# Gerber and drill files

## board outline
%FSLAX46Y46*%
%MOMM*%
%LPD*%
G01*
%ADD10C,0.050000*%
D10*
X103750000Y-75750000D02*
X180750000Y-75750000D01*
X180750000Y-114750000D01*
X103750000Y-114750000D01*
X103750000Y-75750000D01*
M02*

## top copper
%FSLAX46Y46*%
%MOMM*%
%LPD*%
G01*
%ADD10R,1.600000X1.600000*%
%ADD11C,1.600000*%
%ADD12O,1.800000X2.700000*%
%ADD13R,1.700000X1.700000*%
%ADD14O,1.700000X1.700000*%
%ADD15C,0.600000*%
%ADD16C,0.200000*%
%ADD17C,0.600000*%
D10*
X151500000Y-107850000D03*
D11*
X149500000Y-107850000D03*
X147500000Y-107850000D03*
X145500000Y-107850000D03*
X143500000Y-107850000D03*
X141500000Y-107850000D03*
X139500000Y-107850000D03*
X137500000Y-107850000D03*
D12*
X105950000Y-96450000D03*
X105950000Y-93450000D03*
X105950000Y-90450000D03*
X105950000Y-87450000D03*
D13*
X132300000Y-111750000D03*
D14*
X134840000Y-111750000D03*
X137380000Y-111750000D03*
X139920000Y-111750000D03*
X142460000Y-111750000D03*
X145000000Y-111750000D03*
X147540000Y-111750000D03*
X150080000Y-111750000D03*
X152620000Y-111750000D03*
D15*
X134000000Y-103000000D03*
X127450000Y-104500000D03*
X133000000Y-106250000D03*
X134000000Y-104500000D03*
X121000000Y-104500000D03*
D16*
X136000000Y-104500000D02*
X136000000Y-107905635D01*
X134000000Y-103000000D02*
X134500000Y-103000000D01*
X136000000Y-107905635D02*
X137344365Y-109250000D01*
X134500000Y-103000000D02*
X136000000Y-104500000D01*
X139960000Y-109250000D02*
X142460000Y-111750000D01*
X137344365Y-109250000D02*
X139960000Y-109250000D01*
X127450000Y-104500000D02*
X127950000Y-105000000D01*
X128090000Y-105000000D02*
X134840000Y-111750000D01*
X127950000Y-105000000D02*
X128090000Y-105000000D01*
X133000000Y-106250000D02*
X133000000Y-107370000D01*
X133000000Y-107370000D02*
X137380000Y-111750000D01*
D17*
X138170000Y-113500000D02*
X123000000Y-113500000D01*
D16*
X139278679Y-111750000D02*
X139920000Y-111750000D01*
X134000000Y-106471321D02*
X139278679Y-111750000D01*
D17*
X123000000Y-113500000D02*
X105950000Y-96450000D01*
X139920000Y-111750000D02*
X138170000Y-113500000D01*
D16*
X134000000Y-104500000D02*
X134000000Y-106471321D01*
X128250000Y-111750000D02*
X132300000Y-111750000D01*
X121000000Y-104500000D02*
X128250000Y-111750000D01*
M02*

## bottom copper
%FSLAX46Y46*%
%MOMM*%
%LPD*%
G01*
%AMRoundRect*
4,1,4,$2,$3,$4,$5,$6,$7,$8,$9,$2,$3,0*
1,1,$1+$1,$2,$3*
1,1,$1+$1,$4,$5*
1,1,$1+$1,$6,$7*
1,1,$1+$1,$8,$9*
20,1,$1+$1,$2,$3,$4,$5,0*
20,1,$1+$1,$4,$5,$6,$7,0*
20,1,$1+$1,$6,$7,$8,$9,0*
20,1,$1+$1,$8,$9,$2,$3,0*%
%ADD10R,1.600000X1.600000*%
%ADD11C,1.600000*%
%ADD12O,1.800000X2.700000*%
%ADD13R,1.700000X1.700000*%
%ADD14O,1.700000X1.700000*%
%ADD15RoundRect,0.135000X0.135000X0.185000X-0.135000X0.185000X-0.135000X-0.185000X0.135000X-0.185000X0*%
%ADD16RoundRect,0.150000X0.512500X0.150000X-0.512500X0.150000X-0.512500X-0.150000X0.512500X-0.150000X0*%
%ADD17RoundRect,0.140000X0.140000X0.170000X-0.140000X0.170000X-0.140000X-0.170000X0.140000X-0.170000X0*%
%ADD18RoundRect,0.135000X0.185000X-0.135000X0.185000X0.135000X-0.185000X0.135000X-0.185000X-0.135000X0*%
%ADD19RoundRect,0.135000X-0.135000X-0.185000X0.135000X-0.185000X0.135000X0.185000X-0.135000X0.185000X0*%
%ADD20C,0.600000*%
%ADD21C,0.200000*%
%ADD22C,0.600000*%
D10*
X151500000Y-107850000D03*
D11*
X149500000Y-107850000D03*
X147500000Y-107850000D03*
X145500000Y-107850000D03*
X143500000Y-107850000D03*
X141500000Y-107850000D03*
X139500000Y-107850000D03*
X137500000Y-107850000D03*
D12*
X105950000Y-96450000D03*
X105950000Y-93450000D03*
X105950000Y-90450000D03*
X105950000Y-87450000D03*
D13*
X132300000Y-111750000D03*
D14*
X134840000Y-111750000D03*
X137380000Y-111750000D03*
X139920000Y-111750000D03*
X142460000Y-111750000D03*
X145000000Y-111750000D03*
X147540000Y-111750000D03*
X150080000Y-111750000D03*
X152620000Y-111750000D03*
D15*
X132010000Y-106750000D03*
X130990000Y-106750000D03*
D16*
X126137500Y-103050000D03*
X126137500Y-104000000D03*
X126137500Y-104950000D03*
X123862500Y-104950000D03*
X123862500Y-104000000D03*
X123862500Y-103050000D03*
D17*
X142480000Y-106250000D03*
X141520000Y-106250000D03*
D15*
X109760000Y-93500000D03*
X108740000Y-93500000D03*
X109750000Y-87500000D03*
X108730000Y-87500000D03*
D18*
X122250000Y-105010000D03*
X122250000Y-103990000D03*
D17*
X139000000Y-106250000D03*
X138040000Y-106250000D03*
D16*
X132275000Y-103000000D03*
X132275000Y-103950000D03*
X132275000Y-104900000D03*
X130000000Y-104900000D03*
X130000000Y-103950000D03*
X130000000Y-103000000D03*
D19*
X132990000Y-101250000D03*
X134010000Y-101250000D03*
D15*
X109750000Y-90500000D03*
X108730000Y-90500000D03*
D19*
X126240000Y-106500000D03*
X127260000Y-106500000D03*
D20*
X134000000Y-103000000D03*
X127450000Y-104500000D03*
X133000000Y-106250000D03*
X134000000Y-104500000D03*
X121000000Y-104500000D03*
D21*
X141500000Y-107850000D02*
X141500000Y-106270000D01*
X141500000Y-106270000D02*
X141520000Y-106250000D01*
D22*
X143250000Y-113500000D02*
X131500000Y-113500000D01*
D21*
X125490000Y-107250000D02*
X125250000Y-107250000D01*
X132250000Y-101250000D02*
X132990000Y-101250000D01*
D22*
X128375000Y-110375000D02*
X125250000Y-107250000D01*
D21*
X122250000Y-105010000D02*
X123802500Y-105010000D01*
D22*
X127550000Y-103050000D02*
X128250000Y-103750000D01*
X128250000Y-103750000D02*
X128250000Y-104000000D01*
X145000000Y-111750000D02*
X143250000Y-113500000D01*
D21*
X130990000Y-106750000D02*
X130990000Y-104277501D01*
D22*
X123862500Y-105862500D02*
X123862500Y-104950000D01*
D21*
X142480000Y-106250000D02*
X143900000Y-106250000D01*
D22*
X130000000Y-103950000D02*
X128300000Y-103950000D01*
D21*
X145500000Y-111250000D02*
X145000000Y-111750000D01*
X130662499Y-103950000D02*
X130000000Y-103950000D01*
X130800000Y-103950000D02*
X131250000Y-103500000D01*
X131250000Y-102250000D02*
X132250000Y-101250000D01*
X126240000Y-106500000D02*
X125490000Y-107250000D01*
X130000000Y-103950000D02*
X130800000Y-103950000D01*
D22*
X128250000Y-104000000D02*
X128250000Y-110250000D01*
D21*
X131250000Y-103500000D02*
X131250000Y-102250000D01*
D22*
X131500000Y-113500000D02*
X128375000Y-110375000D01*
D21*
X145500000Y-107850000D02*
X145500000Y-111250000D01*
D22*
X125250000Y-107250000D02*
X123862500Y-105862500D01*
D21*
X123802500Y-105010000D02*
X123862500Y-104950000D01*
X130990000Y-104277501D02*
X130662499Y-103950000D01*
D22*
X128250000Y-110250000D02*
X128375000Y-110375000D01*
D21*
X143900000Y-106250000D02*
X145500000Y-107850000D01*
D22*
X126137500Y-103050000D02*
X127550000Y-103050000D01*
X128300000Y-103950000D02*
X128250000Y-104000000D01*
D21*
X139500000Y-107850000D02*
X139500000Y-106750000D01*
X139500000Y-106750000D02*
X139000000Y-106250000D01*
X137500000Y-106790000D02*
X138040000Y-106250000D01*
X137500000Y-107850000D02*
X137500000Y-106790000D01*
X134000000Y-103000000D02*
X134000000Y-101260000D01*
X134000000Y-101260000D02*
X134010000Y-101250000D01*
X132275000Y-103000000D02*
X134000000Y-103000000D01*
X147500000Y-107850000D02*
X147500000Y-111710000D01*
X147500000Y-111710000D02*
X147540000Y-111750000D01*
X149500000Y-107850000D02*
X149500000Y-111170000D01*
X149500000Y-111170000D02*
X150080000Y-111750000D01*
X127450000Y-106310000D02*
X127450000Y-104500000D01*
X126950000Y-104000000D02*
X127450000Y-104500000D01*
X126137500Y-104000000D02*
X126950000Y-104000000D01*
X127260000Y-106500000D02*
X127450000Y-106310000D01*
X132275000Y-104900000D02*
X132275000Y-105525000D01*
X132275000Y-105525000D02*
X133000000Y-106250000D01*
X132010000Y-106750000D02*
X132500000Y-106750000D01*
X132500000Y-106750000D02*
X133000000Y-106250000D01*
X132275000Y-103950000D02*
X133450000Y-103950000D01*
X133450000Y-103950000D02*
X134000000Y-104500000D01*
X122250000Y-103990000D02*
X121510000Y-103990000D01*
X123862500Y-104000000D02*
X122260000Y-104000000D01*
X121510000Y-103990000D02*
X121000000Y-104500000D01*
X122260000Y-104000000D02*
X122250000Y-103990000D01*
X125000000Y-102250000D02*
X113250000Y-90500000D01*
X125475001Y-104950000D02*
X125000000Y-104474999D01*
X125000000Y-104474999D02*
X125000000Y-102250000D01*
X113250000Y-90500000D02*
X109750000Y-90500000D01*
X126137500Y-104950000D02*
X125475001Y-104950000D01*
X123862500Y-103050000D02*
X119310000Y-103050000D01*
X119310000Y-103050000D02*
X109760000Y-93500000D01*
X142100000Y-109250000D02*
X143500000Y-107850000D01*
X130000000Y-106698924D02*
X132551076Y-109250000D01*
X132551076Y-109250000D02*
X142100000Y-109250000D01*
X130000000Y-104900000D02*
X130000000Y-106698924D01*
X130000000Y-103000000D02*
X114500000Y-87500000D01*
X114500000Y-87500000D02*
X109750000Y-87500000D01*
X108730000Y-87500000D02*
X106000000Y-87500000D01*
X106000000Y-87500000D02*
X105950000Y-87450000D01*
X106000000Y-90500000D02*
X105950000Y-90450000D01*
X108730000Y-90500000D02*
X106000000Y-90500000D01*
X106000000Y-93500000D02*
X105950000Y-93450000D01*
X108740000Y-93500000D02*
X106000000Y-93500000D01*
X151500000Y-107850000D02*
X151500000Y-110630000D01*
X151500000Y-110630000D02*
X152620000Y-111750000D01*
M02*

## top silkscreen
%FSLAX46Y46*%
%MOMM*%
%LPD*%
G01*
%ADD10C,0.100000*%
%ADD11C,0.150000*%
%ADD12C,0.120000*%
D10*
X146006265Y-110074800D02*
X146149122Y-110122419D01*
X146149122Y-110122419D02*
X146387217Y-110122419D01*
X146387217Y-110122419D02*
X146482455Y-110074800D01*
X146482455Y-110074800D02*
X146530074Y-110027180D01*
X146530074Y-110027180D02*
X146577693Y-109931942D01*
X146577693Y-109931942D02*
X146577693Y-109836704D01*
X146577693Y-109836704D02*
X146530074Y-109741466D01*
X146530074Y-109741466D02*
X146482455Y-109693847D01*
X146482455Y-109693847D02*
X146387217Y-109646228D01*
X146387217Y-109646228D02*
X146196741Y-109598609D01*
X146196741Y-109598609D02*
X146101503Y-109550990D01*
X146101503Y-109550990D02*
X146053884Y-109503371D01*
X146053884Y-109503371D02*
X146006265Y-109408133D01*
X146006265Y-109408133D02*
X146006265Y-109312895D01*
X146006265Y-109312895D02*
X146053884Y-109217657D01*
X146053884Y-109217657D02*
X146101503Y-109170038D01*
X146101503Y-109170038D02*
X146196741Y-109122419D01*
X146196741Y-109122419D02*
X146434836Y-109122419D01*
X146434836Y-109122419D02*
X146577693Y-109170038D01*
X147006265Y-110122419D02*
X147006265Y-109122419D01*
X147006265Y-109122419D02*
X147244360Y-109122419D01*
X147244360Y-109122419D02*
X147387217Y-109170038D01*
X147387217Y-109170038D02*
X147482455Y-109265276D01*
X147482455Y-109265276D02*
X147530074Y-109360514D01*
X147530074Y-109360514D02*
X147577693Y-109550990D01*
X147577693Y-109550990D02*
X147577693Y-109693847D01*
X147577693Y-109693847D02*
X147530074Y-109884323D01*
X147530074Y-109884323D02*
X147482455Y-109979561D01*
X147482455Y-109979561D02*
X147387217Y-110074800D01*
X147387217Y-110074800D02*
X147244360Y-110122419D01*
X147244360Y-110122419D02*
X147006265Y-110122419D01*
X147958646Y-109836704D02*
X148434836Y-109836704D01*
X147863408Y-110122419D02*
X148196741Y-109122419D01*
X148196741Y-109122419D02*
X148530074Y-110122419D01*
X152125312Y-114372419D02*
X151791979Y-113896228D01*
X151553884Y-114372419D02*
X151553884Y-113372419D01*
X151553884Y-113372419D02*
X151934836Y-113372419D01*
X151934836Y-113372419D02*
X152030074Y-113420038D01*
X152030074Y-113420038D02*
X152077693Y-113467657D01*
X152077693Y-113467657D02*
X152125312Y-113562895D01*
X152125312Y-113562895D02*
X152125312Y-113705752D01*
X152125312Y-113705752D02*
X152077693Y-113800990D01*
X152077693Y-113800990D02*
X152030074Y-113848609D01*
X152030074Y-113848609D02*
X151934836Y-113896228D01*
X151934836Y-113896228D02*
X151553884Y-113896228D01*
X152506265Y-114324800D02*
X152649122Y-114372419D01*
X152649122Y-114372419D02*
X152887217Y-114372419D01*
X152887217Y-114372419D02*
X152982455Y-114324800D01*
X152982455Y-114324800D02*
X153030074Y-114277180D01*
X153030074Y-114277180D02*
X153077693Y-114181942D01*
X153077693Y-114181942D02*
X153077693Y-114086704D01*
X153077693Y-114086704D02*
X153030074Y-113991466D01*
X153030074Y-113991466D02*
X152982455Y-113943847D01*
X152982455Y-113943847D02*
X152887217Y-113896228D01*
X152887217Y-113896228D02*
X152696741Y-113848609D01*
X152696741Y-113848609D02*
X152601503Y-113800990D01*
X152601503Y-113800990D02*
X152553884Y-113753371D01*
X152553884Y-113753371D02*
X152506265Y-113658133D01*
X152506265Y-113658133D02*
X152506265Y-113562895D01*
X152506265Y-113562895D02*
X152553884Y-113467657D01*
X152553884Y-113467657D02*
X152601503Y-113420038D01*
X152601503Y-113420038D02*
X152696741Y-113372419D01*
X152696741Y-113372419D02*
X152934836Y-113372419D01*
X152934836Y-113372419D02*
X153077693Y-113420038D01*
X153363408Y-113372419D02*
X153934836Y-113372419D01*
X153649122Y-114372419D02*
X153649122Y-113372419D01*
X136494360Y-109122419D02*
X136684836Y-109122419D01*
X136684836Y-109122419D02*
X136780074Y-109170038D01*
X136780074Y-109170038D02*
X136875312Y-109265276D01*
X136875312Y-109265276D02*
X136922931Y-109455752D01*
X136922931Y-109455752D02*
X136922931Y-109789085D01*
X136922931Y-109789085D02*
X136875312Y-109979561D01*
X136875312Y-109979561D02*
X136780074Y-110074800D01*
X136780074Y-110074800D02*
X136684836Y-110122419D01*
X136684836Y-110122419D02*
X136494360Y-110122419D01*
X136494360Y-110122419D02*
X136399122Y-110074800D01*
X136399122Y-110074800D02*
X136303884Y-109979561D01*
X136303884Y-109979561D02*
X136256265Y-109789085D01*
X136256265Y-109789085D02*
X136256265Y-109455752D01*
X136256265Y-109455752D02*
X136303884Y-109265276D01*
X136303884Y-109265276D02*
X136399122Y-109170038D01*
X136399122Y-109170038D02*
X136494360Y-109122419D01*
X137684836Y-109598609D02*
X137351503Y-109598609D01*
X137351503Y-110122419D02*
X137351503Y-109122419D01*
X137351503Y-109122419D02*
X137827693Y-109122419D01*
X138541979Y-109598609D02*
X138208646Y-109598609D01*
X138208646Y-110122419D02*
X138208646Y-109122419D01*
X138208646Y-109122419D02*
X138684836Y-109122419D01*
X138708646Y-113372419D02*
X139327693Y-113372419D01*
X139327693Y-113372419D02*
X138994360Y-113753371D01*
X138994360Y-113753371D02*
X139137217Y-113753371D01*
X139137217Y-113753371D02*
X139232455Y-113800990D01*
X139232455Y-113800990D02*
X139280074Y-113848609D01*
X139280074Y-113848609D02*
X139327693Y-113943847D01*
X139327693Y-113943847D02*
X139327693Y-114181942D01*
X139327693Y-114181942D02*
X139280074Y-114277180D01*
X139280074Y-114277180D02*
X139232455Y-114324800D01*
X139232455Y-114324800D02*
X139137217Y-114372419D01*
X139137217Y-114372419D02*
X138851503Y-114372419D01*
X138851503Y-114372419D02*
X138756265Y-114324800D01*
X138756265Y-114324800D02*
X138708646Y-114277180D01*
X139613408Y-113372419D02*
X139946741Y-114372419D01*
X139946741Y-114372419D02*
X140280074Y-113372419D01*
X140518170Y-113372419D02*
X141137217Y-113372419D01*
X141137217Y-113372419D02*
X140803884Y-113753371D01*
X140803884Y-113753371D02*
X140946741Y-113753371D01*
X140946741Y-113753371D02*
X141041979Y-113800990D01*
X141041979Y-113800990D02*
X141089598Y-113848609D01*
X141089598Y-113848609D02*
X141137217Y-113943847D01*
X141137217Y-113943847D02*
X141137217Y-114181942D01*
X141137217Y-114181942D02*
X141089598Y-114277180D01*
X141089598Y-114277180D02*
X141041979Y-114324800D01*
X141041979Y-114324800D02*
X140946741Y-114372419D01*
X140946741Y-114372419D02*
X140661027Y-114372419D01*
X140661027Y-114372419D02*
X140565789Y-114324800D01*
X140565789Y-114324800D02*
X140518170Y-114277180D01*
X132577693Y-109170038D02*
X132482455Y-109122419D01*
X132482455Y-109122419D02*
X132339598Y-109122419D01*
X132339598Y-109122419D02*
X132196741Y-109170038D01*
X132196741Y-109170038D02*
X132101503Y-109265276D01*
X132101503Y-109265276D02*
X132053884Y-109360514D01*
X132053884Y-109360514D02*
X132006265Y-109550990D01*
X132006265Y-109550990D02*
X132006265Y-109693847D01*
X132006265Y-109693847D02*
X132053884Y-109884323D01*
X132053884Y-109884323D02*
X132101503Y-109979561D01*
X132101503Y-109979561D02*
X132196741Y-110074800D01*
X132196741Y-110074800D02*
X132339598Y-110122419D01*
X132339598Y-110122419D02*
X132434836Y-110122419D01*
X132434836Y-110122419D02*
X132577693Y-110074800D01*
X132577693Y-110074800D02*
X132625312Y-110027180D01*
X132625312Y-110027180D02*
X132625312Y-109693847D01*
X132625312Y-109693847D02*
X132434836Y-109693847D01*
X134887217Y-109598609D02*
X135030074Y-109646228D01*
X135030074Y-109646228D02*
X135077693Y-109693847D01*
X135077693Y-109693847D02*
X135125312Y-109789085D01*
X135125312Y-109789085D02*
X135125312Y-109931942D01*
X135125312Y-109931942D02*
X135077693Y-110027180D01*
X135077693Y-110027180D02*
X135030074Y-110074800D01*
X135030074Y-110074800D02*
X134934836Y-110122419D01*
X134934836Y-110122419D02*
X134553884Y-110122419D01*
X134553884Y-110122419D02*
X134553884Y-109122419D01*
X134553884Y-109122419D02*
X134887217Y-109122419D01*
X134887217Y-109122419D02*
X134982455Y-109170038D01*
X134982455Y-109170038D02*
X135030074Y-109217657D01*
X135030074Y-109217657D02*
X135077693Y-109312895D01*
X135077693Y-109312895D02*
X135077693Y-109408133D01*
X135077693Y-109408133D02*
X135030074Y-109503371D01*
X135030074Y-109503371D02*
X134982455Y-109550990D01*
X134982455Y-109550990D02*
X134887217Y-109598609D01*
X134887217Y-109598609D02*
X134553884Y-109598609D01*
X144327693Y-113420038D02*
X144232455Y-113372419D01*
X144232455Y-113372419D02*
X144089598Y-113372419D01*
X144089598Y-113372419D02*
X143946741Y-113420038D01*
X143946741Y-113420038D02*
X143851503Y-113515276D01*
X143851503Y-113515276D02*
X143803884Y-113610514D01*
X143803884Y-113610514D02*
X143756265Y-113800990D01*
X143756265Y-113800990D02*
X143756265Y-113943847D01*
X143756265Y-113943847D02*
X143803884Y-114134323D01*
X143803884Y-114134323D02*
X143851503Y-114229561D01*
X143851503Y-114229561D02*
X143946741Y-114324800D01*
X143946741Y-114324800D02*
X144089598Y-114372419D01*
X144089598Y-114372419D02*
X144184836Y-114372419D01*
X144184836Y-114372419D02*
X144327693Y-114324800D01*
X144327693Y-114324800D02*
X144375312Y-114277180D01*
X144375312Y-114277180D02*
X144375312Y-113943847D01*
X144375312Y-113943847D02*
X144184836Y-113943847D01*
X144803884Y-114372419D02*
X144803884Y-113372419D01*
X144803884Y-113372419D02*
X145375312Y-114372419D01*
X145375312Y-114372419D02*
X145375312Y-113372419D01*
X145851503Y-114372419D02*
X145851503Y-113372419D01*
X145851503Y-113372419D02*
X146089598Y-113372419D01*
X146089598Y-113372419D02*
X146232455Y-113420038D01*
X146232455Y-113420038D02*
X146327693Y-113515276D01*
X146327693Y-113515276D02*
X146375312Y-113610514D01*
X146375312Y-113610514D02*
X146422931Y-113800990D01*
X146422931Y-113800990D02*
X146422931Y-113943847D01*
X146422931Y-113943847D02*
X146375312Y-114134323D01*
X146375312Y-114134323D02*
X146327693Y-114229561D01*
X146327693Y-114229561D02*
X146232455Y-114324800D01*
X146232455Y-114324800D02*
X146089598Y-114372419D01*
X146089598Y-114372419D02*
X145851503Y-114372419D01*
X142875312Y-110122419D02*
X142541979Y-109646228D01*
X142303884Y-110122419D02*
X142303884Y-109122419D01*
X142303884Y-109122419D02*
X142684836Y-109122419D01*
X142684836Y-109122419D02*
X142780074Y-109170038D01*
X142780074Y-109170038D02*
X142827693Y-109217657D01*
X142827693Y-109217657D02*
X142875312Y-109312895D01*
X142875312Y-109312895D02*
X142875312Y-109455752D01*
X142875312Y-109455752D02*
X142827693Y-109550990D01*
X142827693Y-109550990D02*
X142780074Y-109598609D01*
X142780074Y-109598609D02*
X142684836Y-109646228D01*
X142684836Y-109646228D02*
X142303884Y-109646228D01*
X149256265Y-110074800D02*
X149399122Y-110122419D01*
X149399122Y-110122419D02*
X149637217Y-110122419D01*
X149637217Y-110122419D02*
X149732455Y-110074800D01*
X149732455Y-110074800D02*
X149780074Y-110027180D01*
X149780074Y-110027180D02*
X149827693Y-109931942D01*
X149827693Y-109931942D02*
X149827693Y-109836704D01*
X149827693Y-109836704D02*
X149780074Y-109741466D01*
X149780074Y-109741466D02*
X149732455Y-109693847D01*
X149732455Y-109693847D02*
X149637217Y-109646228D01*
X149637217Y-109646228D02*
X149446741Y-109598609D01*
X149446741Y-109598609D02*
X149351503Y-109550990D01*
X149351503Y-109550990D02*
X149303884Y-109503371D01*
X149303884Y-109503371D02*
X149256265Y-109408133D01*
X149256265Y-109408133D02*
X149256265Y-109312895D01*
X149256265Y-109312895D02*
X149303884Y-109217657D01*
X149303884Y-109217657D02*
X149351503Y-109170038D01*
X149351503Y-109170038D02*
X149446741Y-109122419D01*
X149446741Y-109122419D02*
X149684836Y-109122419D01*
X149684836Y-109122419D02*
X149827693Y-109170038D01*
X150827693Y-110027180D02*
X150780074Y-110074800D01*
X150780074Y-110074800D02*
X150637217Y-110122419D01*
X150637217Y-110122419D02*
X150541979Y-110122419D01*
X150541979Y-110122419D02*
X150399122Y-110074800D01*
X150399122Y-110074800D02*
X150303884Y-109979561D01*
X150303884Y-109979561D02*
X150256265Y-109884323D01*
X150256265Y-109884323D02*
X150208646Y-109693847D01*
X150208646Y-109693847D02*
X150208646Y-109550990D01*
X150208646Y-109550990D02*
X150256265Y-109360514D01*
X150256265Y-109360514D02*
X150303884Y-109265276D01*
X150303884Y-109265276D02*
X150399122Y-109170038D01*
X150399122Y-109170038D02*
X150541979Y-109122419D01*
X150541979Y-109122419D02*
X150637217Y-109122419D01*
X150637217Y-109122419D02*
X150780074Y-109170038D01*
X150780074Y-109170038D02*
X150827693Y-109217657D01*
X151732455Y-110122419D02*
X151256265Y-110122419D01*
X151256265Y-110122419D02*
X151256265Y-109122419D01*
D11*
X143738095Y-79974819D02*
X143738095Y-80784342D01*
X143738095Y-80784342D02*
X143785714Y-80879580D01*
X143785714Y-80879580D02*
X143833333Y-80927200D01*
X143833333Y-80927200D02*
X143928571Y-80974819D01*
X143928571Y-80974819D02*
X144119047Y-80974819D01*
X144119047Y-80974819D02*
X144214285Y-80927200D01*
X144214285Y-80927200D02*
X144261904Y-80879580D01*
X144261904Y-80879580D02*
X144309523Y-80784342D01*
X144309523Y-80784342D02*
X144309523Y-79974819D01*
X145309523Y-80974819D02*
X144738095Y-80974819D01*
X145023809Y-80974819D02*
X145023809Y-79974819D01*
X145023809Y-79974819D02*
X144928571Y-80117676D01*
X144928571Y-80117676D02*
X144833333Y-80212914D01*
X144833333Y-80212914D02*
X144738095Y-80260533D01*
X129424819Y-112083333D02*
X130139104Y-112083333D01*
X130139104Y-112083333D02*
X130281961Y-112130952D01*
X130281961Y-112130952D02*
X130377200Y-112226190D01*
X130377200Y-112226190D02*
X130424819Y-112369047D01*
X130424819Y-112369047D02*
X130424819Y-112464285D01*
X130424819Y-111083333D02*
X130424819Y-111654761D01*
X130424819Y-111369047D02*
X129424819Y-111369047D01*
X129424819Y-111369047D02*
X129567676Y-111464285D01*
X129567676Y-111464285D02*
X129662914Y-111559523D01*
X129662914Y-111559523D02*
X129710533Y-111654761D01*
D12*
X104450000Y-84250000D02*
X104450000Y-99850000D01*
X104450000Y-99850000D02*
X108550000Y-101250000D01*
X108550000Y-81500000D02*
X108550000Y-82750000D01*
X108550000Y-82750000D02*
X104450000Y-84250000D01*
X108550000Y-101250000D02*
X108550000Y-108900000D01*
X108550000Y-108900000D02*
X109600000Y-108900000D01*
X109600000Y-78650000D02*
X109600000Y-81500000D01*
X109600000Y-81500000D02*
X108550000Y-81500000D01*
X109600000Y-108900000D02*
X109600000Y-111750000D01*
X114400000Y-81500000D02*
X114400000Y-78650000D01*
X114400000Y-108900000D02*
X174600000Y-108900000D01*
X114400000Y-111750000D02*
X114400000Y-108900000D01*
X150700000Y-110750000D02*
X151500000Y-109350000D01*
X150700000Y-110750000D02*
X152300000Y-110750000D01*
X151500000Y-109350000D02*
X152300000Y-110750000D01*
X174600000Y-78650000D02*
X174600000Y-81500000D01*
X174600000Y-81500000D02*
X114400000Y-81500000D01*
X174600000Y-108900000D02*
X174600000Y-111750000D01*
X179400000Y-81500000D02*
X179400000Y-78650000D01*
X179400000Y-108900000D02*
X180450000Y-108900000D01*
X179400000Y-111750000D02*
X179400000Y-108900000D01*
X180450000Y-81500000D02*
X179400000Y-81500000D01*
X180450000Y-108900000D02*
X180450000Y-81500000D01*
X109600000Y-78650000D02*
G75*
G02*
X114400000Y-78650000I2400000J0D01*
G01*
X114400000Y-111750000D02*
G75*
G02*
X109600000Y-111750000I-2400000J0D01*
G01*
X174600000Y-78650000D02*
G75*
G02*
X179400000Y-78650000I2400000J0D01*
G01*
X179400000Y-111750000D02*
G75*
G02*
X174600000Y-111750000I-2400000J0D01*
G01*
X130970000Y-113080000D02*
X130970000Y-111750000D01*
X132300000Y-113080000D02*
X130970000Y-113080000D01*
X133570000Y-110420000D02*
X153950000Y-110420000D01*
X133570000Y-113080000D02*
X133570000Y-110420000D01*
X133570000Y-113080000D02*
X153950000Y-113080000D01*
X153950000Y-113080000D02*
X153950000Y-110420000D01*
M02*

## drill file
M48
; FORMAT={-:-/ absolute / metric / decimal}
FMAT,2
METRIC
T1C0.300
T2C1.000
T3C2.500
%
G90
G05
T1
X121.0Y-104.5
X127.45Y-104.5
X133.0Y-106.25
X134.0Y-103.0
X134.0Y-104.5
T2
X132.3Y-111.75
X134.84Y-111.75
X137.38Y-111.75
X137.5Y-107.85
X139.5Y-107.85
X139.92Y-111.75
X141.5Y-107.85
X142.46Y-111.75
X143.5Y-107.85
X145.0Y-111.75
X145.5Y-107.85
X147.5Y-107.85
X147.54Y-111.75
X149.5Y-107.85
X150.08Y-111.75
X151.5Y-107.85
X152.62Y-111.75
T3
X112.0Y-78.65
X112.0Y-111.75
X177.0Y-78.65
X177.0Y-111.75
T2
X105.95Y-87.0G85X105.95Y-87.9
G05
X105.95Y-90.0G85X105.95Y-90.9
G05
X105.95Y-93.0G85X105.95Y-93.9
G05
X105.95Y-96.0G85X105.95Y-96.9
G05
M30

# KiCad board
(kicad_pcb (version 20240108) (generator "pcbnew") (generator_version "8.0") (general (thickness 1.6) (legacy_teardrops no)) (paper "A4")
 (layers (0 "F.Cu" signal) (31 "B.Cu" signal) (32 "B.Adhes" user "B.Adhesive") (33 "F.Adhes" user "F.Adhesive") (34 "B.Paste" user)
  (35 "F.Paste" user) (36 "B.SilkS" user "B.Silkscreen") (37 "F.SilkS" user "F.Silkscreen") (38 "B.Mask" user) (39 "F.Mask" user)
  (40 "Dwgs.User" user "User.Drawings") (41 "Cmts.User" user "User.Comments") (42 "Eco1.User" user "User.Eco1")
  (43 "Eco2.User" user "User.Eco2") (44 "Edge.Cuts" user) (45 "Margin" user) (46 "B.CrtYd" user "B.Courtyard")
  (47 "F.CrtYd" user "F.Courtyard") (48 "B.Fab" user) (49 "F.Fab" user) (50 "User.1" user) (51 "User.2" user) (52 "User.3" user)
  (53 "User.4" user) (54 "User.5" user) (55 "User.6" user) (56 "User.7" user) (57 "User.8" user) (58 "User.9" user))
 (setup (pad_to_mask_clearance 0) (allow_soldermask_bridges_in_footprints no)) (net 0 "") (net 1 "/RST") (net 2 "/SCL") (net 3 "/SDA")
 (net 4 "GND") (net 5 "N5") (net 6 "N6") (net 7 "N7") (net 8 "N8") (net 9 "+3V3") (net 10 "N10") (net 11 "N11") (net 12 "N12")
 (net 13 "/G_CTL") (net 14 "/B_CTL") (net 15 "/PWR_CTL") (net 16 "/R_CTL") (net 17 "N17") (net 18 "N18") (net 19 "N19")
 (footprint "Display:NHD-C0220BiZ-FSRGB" (layer "F.Cu") (at 144.5 91.95)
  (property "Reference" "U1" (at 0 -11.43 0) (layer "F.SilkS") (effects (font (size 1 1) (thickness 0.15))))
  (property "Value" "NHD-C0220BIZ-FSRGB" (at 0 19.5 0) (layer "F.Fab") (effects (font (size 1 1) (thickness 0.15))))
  (fp_line (start -40.05 -7.7) (end -40.05 7.9) (stroke (width 0.12) (type solid)) (layer "F.SilkS"))
  (fp_line (start -40.05 7.9) (end -35.95 9.3) (stroke (width 0.12) (type solid)) (layer "F.SilkS"))
  (fp_line (start -35.95 -10.45) (end -35.95 -9.2) (stroke (width 0.12) (type solid)) (layer "F.SilkS"))
  (fp_line (start -35.95 -9.2) (end -40.05 -7.7) (stroke (width 0.12) (type solid)) (layer "F.SilkS"))
  (fp_line (start -35.95 9.3) (end -35.95 16.95) (stroke (width 0.12) (type solid)) (layer "F.SilkS"))
  (fp_line (start -35.95 16.95) (end -34.9 16.95) (stroke (width 0.12) (type solid)) (layer "F.SilkS"))
  (fp_line (start -34.9 -13.3) (end -34.9 -10.45) (stroke (width 0.12) (type solid)) (layer "F.SilkS"))
  (fp_line (start -34.9 -10.45) (end -35.95 -10.45) (stroke (width 0.12) (type solid)) (layer "F.SilkS"))
  (fp_line (start -34.9 16.95) (end -34.9 19.8) (stroke (width 0.12) (type solid)) (layer "F.SilkS"))
  (fp_line (start -30.1 -10.45) (end -30.1 -13.3) (stroke (width 0.12) (type solid)) (layer "F.SilkS"))
  (fp_line (start -30.1 16.95) (end 30.1 16.95) (stroke (width 0.12) (type solid)) (layer "F.SilkS"))
  (fp_line (start -30.1 19.8) (end -30.1 16.95) (stroke (width 0.12) (type solid)) (layer "F.SilkS"))
  (fp_line (start 6.2 18.8) (end 7 17.4) (stroke (width 0.12) (type solid)) (layer "F.SilkS"))
  (fp_line (start 6.2 18.8) (end 7.8 18.8) (stroke (width 0.12) (type solid)) (layer "F.SilkS"))
  (fp_line (start 7 17.4) (end 7.8 18.8) (stroke (width 0.12) (type solid)) (layer "F.SilkS"))
  (fp_line (start 30.1 -13.3) (end 30.1 -10.45) (stroke (width 0.12) (type solid)) (layer "F.SilkS"))
  (fp_line (start 30.1 -10.45) (end -30.1 -10.45) (stroke (width 0.12) (type solid)) (layer "F.SilkS"))
  (fp_line (start 30.1 16.95) (end 30.1 19.8) (stroke (width 0.12) (type solid)) (layer "F.SilkS"))
  (fp_line (start 34.9 -10.45) (end 34.9 -13.3) (stroke (width 0.12) (type solid)) (layer "F.SilkS"))
  (fp_line (start 34.9 16.95) (end 35.95 16.95) (stroke (width 0.12) (type solid)) (layer "F.SilkS"))
  (fp_line (start 34.9 19.8) (end 34.9 16.95) (stroke (width 0.12) (type solid)) (layer "F.SilkS"))
  (fp_line (start 35.95 -10.45) (end 34.9 -10.45) (stroke (width 0.12) (type solid)) (layer "F.SilkS"))
  (fp_line (start 35.95 16.95) (end 35.95 -10.45) (stroke (width 0.12) (type solid)) (layer "F.SilkS"))
  (fp_arc (start -34.9 -13.3) (mid -32.5 -15.7) (end -30.1 -13.3) (stroke (width 0.12) (type solid)) (layer "F.SilkS"))
  (fp_arc (start -30.1 19.8) (mid -32.5 22.2) (end -34.9 19.8) (stroke (width 0.12) (type solid)) (layer "F.SilkS"))
  (fp_arc (start 30.1 -13.3) (mid 32.5 -15.7) (end 34.9 -13.3) (stroke (width 0.12) (type solid)) (layer "F.SilkS"))
  (fp_arc (start 34.9 19.8) (mid 32.5 22.2) (end 30.1 19.8) (stroke (width 0.12) (type solid)) (layer "F.SilkS"))
  (pad "" np_thru_hole circle (at -32.5 -13.3) (size 2.5 2.5) (drill 2.5) (layers "*.Cu" "*.Mask"))
  (pad "" np_thru_hole circle (at -32.5 19.8) (size 2.5 2.5) (drill 2.5) (layers "*.Cu" "*.Mask"))
  (pad "" np_thru_hole circle (at 32.5 -13.3) (size 2.5 2.5) (drill 2.5) (layers "*.Cu" "*.Mask"))
  (pad "" np_thru_hole circle (at 32.5 19.8) (size 2.5 2.5) (drill 2.5) (layers "*.Cu" "*.Mask"))
  (pad "1" thru_hole rect (at 7 15.9) (size 1.6 1.6) (drill 1) (layers "*.Cu" "*.Mask") (remove_unused_layers no) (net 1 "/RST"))
  (pad "2" thru_hole circle (at 5 15.9) (size 1.6 1.6) (drill 1) (layers "*.Cu" "*.Mask") (remove_unused_layers no) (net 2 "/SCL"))
  (pad "3" thru_hole circle (at 3 15.9) (size 1.6 1.6) (drill 1) (layers "*.Cu" "*.Mask") (remove_unused_layers no) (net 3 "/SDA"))
  (pad "4" thru_hole circle (at 1 15.9) (size 1.6 1.6) (drill 1) (layers "*.Cu" "*.Mask") (remove_unused_layers no) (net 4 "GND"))
  (pad "5" thru_hole circle (at -1 15.9) (size 1.6 1.6) (drill 1) (layers "*.Cu" "*.Mask") (remove_unused_layers no) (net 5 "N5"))
  (pad "6" thru_hole circle (at -3 15.9) (size 1.6 1.6) (drill 1) (layers "*.Cu" "*.Mask") (remove_unused_layers no) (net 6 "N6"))
  (pad "7" thru_hole circle (at -5 15.9) (size 1.6 1.6) (drill 1) (layers "*.Cu" "*.Mask") (remove_unused_layers no) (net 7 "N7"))
  (pad "8" thru_hole circle (at -7 15.9) (size 1.6 1.6) (drill 1) (layers "*.Cu" "*.Mask") (remove_unused_layers no) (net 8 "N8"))
  (pad "9" thru_hole oval (at -38.55 4.5) (size 1.8 2.7) (drill oval 1 1.9) (layers "*.Cu" "*.Mask") (remove_unused_layers no)
   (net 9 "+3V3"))
  (pad "10" thru_hole oval (at -38.55 1.5) (size 1.8 2.7) (drill oval 1 1.9) (layers "*.Cu" "*.Mask") (remove_unused_layers no)
   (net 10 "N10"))
  (pad "11" thru_hole oval (at -38.55 -1.5) (size 1.8 2.7) (drill oval 1 1.9) (layers "*.Cu" "*.Mask") (remove_unused_layers no)
   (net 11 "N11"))
  (pad "12" thru_hole oval (at -38.55 -4.5) (size 1.8 2.7) (drill oval 1 1.9) (layers "*.Cu" "*.Mask") (remove_unused_layers no)
   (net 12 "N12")))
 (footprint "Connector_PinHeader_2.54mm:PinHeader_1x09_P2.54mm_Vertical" (layer "F.Cu") (at 132.3 111.75 90)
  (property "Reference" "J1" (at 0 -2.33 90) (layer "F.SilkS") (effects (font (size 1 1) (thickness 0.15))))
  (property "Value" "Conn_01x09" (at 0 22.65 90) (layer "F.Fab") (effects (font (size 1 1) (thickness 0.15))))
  (fp_line (start -1.33 -1.33) (end 0 -1.33) (stroke (width 0.12) (type solid)) (layer "F.SilkS"))
  (fp_line (start -1.33 0) (end -1.33 -1.33) (stroke (width 0.12) (type solid)) (layer "F.SilkS"))
  (fp_line (start 1.33 1.27) (end 1.33 21.65) (stroke (width 0.12) (type solid)) (layer "F.SilkS"))
  (fp_line (start -1.33 1.27) (end 1.33 1.27) (stroke (width 0.12) (type solid)) (layer "F.SilkS"))
  (fp_line (start -1.33 1.27) (end -1.33 21.65) (stroke (width 0.12) (type solid)) (layer "F.SilkS"))
  (fp_line (start -1.33 21.65) (end 1.33 21.65) (stroke (width 0.12) (type solid)) (layer "F.SilkS"))
  (pad "1" thru_hole rect (at 0 0 90) (size 1.7 1.7) (drill 1) (layers "*.Cu" "*.Mask") (remove_unused_layers no) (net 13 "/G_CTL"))
  (pad "2" thru_hole oval (at 0 2.54 90) (size 1.7 1.7) (drill 1) (layers "*.Cu" "*.Mask") (remove_unused_layers no) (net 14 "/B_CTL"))
  (pad "3" thru_hole oval (at 0 5.08 90) (size 1.7 1.7) (drill 1) (layers "*.Cu" "*.Mask") (remove_unused_layers no) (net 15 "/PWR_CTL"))
  (pad "4" thru_hole oval (at 0 7.62 90) (size 1.7 1.7) (drill 1) (layers "*.Cu" "*.Mask") (remove_unused_layers no) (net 9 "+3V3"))
  (pad "5" thru_hole oval (at 0 10.16 90) (size 1.7 1.7) (drill 1) (layers "*.Cu" "*.Mask") (remove_unused_layers no) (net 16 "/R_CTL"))
  (pad "6" thru_hole oval (at 0 12.7 90) (size 1.7 1.7) (drill 1) (layers "*.Cu" "*.Mask") (remove_unused_layers no) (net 4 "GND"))
  (pad "7" thru_hole oval (at 0 15.24 90) (size 1.7 1.7) (drill 1) (layers "*.Cu" "*.Mask") (remove_unused_layers no) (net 3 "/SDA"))
  (pad "8" thru_hole oval (at 0 17.78 90) (size 1.7 1.7) (drill 1) (layers "*.Cu" "*.Mask") (remove_unused_layers no) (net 2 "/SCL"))
  (pad "9" thru_hole oval (at 0 20.32 90) (size 1.7 1.7) (drill 1) (layers "*.Cu" "*.Mask") (remove_unused_layers no) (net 1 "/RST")))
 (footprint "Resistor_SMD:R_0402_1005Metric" (layer "B.Cu") (at 131.5 106.75 180)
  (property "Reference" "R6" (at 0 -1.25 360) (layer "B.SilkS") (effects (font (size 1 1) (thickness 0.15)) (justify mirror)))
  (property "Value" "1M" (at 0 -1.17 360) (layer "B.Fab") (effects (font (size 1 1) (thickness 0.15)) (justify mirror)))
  (pad "1" smd roundrect (at -0.51 0 180) (size 0.54 0.64) (layers "B.Cu" "B.Paste" "B.Mask") (roundrect_rratio 0.25) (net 15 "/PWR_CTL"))
  (pad "2" smd roundrect (at 0.51 0 180) (size 0.54 0.64) (layers "B.Cu" "B.Paste" "B.Mask") (roundrect_rratio 0.25) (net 4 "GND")))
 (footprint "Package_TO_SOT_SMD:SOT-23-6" (layer "B.Cu") (at 125 104 180)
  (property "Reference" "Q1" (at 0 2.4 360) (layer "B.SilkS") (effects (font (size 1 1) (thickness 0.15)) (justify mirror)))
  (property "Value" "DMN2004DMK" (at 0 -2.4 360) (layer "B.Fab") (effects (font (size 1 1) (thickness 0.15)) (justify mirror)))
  (pad "1" smd roundrect (at -1.1375 0.95 180) (size 1.325 0.6) (layers "B.Cu" "B.Paste" "B.Mask") (roundrect_rratio 0.25) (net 4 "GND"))
  (pad "2" smd roundrect (at -1.1375 0 180) (size 1.325 0.6) (layers "B.Cu" "B.Paste" "B.Mask") (roundrect_rratio 0.25) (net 14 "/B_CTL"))
  (pad "3" smd roundrect (at -1.1375 -0.95 180) (size 1.325 0.6) (layers "B.Cu" "B.Paste" "B.Mask") (roundrect_rratio 0.25) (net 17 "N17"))
  (pad "4" smd roundrect (at 1.1375 -0.95 180) (size 1.325 0.6) (layers "B.Cu" "B.Paste" "B.Mask") (roundrect_rratio 0.25) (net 4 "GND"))
  (pad "5" smd roundrect (at 1.1375 0 180) (size 1.325 0.6) (layers "B.Cu" "B.Paste" "B.Mask") (roundrect_rratio 0.25) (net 13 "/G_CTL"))
  (pad "6" smd roundrect (at 1.1375 0.95 180) (size 1.325 0.6) (layers "B.Cu" "B.Paste" "B.Mask") (roundrect_rratio 0.25) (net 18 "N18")))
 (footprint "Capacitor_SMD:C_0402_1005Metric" (layer "B.Cu") (at 142 106.25 180)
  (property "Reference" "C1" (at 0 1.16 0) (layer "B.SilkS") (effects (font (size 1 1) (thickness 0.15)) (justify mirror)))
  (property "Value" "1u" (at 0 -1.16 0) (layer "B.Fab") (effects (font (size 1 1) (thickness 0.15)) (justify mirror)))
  (pad "1" smd roundrect (at -0.48 0 180) (size 0.56 0.62) (layers "B.Cu" "B.Paste" "B.Mask") (roundrect_rratio 0.25) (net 4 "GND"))
  (pad "2" smd roundrect (at 0.48 0 180) (size 0.56 0.62) (layers "B.Cu" "B.Paste" "B.Mask") (roundrect_rratio 0.25) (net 6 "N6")))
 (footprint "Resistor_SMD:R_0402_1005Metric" (layer "B.Cu") (at 109.25 93.5 180)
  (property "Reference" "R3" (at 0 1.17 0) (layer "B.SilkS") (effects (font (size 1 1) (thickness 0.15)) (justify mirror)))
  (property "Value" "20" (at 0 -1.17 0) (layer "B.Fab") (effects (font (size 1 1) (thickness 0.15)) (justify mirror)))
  (pad "1" smd roundrect (at -0.51 0 180) (size 0.54 0.64) (layers "B.Cu" "B.Paste" "B.Mask") (roundrect_rratio 0.25) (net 18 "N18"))
  (pad "2" smd roundrect (at 0.51 0 180) (size 0.54 0.64) (layers "B.Cu" "B.Paste" "B.Mask") (roundrect_rratio 0.25) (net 10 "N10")))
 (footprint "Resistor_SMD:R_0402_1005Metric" (layer "B.Cu") (at 109.24 87.5 180)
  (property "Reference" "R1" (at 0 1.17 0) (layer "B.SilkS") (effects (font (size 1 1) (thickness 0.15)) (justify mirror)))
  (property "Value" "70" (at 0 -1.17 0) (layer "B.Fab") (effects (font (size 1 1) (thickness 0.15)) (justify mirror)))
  (pad "1" smd roundrect (at -0.51 0 180) (size 0.54 0.64) (layers "B.Cu" "B.Paste" "B.Mask") (roundrect_rratio 0.25) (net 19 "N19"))
  (pad "2" smd roundrect (at 0.51 0 180) (size 0.54 0.64) (layers "B.Cu" "B.Paste" "B.Mask") (roundrect_rratio 0.25) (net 12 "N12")))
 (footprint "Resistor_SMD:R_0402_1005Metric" (layer "B.Cu") (at 122.25 104.5 90)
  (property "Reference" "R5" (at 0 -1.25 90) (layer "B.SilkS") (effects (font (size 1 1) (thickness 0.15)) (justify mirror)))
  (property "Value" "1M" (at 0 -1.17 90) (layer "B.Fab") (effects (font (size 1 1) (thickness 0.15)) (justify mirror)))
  (pad "1" smd roundrect (at -0.51 0 90) (size 0.54 0.64) (layers "B.Cu" "B.Paste" "B.Mask") (roundrect_rratio 0.25) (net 4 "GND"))
  (pad "2" smd roundrect (at 0.51 0 90) (size 0.54 0.64) (layers "B.Cu" "B.Paste" "B.Mask") (roundrect_rratio 0.25) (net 13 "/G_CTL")))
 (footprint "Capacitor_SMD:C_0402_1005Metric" (layer "B.Cu") (at 138.52 106.25 180)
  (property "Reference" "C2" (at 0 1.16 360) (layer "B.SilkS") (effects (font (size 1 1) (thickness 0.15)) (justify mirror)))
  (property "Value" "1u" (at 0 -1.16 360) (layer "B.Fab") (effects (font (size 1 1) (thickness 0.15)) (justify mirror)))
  (pad "1" smd roundrect (at -0.48 0 180) (size 0.56 0.62) (layers "B.Cu" "B.Paste" "B.Mask") (roundrect_rratio 0.25) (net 7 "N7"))
  (pad "2" smd roundrect (at 0.48 0 180) (size 0.56 0.62) (layers "B.Cu" "B.Paste" "B.Mask") (roundrect_rratio 0.25) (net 8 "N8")))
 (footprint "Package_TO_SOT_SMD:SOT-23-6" (layer "B.Cu") (at 131.1375 103.95 180)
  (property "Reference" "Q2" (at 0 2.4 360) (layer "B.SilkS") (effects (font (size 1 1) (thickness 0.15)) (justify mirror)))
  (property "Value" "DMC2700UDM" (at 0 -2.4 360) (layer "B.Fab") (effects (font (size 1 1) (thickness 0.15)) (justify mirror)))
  (pad "1" smd roundrect (at -1.1375 0.95 180) (size 1.325 0.6) (layers "B.Cu" "B.Paste" "B.Mask") (roundrect_rratio 0.25) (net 16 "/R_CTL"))
  (pad "2" smd roundrect (at -1.1375 0 180) (size 1.325 0.6) (layers "B.Cu" "B.Paste" "B.Mask") (roundrect_rratio 0.25) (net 9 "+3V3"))
  (pad "3" smd roundrect (at -1.1375 -0.95 180) (size 1.325 0.6) (layers "B.Cu" "B.Paste" "B.Mask") (roundrect_rratio 0.25)
   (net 15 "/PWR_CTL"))
  (pad "4" smd roundrect (at 1.1375 -0.95 180) (size 1.325 0.6) (layers "B.Cu" "B.Paste" "B.Mask") (roundrect_rratio 0.25) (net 5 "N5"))
  (pad "5" smd roundrect (at 1.1375 0 180) (size 1.325 0.6) (layers "B.Cu" "B.Paste" "B.Mask") (roundrect_rratio 0.25) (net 4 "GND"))
  (pad "6" smd roundrect (at 1.1375 0.95 180) (size 1.325 0.6) (layers "B.Cu" "B.Paste" "B.Mask") (roundrect_rratio 0.25) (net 19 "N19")))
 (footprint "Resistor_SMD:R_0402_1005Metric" (layer "B.Cu") (at 133.5 101.25)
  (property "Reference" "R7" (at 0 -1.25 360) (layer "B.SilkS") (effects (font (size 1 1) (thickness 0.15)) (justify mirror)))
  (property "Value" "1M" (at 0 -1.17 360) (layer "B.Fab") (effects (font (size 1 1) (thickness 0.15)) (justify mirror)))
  (pad "1" smd roundrect (at -0.51 0) (size 0.54 0.64) (layers "B.Cu" "B.Paste" "B.Mask") (roundrect_rratio 0.25) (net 4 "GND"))
  (pad "2" smd roundrect (at 0.51 0) (size 0.54 0.64) (layers "B.Cu" "B.Paste" "B.Mask") (roundrect_rratio 0.25) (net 16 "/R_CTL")))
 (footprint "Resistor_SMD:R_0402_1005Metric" (layer "B.Cu") (at 109.24 90.5 180)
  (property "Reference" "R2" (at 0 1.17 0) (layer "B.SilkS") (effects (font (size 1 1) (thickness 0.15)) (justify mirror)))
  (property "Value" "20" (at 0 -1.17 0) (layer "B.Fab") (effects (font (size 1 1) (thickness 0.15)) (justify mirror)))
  (pad "1" smd roundrect (at -0.51 0 180) (size 0.54 0.64) (layers "B.Cu" "B.Paste" "B.Mask") (roundrect_rratio 0.25) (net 17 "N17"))
  (pad "2" smd roundrect (at 0.51 0 180) (size 0.54 0.64) (layers "B.Cu" "B.Paste" "B.Mask") (roundrect_rratio 0.25) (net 11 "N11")))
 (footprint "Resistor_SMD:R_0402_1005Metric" (layer "B.Cu") (at 126.75 106.5)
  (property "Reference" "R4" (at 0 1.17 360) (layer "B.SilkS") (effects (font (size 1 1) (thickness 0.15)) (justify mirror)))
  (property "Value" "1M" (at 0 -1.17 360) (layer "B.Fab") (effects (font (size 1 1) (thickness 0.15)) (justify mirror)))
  (pad "1" smd roundrect (at -0.51 0) (size 0.54 0.64) (layers "B.Cu" "B.Paste" "B.Mask") (roundrect_rratio 0.25) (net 4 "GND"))
  (pad "2" smd roundrect (at 0.51 0) (size 0.54 0.64) (layers "B.Cu" "B.Paste" "B.Mask") (roundrect_rratio 0.25) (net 14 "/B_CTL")))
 (gr_rect (start 103.75 75.75) (end 180.75 114.75) (stroke (width 0.05) (type default)) (fill none) (layer "Edge.Cuts"))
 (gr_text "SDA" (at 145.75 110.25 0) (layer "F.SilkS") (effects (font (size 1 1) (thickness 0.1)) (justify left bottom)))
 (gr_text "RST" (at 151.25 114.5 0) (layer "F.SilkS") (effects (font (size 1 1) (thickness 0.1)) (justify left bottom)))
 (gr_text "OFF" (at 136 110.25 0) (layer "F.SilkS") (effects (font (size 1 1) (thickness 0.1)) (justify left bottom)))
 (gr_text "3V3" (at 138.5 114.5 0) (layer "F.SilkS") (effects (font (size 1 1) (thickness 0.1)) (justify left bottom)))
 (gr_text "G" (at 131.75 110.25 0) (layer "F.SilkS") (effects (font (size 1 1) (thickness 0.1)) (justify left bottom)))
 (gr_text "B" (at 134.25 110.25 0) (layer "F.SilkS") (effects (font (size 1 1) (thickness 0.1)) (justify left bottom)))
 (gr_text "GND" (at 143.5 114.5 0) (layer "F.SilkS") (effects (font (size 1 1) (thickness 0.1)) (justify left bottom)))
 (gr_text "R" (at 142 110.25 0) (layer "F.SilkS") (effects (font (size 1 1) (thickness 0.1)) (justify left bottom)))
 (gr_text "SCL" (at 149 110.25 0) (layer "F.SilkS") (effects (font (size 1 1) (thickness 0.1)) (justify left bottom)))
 (segment (start 141.5 107.85) (end 141.5 106.27) (width 0.2) (layer "B.Cu") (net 6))
 (segment (start 141.5 106.27) (end 141.52 106.25) (width 0.2) (layer "B.Cu") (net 6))
 (segment (start 143.25 113.5) (end 131.5 113.5) (width 0.6) (layer "B.Cu") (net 4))
 (segment (start 125.49 107.25) (end 125.25 107.25) (width 0.2) (layer "B.Cu") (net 4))
 (segment (start 132.25 101.25) (end 132.99 101.25) (width 0.2) (layer "B.Cu") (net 4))
 (segment (start 128.375 110.375) (end 125.25 107.25) (width 0.6) (layer "B.Cu") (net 4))
 (segment (start 122.25 105.01) (end 123.8025 105.01) (width 0.2) (layer "B.Cu") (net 4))
 (segment (start 127.55 103.05) (end 128.25 103.75) (width 0.6) (layer "B.Cu") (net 4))
 (segment (start 128.25 103.75) (end 128.25 104) (width 0.6) (layer "B.Cu") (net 4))
 (segment (start 145 111.75) (end 143.25 113.5) (width 0.6) (layer "B.Cu") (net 4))
 (segment (start 130.99 106.75) (end 130.99 104.277501) (width 0.2) (layer "B.Cu") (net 4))
 (segment (start 123.8625 105.8625) (end 123.8625 104.95) (width 0.6) (layer "B.Cu") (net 4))
 (segment (start 142.48 106.25) (end 143.9 106.25) (width 0.2) (layer "B.Cu") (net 4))
 (segment (start 130 103.95) (end 128.3 103.95) (width 0.6) (layer "B.Cu") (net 4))
 (segment (start 145.5 111.25) (end 145 111.75) (width 0.2) (layer "B.Cu") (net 4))
 (segment (start 130.662499 103.95) (end 130 103.95) (width 0.2) (layer "B.Cu") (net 4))
 (segment (start 130.8 103.95) (end 131.25 103.5) (width 0.2) (layer "B.Cu") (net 4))
 (segment (start 131.25 102.25) (end 132.25 101.25) (width 0.2) (layer "B.Cu") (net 4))
 (segment (start 126.24 106.5) (end 125.49 107.25) (width 0.2) (layer "B.Cu") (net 4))
 (segment (start 130 103.95) (end 130.8 103.95) (width 0.2) (layer "B.Cu") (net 4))
 (segment (start 128.25 104) (end 128.25 110.25) (width 0.6) (layer "B.Cu") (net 4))
 (segment (start 131.25 103.5) (end 131.25 102.25) (width 0.2) (layer "B.Cu") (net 4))
 (segment (start 131.5 113.5) (end 128.375 110.375) (width 0.6) (layer "B.Cu") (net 4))
 (segment (start 145.5 107.85) (end 145.5 111.25) (width 0.2) (layer "B.Cu") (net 4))
 (segment (start 125.25 107.25) (end 123.8625 105.8625) (width 0.6) (layer "B.Cu") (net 4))
 (segment (start 123.8025 105.01) (end 123.8625 104.95) (width 0.2) (layer "B.Cu") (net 4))
 (segment (start 130.99 104.277501) (end 130.662499 103.95) (width 0.2) (layer "B.Cu") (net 4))
 (segment (start 128.25 110.25) (end 128.375 110.375) (width 0.6) (layer "B.Cu") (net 4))
 (segment (start 143.9 106.25) (end 145.5 107.85) (width 0.2) (layer "B.Cu") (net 4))
 (segment (start 126.1375 103.05) (end 127.55 103.05) (width 0.6) (layer "B.Cu") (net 4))
 (segment (start 128.3 103.95) (end 128.25 104) (width 0.6) (layer "B.Cu") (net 4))
 (segment (start 139.5 107.85) (end 139.5 106.75) (width 0.2) (layer "B.Cu") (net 7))
 (segment (start 139.5 106.75) (end 139 106.25) (width 0.2) (layer "B.Cu") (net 7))
 (segment (start 137.5 106.79) (end 138.04 106.25) (width 0.2) (layer "B.Cu") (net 8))
 (segment (start 137.5 107.85) (end 137.5 106.79) (width 0.2) (layer "B.Cu") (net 8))
 (segment (start 136 104.5) (end 136 107.905635) (width 0.2) (layer "F.Cu") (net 16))
 (segment (start 134 103) (end 134.5 103) (width 0.2) (layer "F.Cu") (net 16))
 (segment (start 136 107.905635) (end 137.344365 109.25) (width 0.2) (layer "F.Cu") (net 16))
 (segment (start 134.5 103) (end 136 104.5) (width 0.2) (layer "F.Cu") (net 16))
 (segment (start 139.96 109.25) (end 142.46 111.75) (width 0.2) (layer "F.Cu") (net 16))
 (segment (start 137.344365 109.25) (end 139.96 109.25) (width 0.2) (layer "F.Cu") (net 16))
 (via (at 134 103) (size 0.6) (drill 0.3) (layers "F.Cu" "B.Cu") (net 16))
 (segment (start 134 103) (end 134 101.26) (width 0.2) (layer "B.Cu") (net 16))
 (segment (start 134 101.26) (end 134.01 101.25) (width 0.2) (layer "B.Cu") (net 16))
 (segment (start 132.275 103) (end 134 103) (width 0.2) (layer "B.Cu") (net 16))
 (segment (start 147.5 107.85) (end 147.5 111.71) (width 0.2) (layer "B.Cu") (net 3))
 (segment (start 147.5 111.71) (end 147.54 111.75) (width 0.2) (layer "B.Cu") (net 3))
 (segment (start 149.5 107.85) (end 149.5 111.17) (width 0.2) (layer "B.Cu") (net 2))
 (segment (start 149.5 111.17) (end 150.08 111.75) (width 0.2) (layer "B.Cu") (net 2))
 (segment (start 127.45 104.5) (end 127.95 105) (width 0.2) (layer "F.Cu") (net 14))
 (segment (start 128.09 105) (end 134.84 111.75) (width 0.2) (layer "F.Cu") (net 14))
 (segment (start 127.95 105) (end 128.09 105) (width 0.2) (layer "F.Cu") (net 14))
 (via (at 127.45 104.5) (size 0.6) (drill 0.3) (layers "F.Cu" "B.Cu") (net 14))
 (segment (start 127.45 106.31) (end 127.45 104.5) (width 0.2) (layer "B.Cu") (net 14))
 (segment (start 126.95 104) (end 127.45 104.5) (width 0.2) (layer "B.Cu") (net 14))
 (segment (start 126.1375 104) (end 126.95 104) (width 0.2) (layer "B.Cu") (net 14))
 (segment (start 127.26 106.5) (end 127.45 106.31) (width 0.2) (layer "B.Cu") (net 14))
 (segment (start 133 106.25) (end 133 107.37) (width 0.2) (layer "F.Cu") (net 15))
 (segment (start 133 107.37) (end 137.38 111.75) (width 0.2) (layer "F.Cu") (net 15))
 (via (at 133 106.25) (size 0.6) (drill 0.3) (layers "F.Cu" "B.Cu") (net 15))
 (segment (start 132.275 104.9) (end 132.275 105.525) (width 0.2) (layer "B.Cu") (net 15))
 (segment (start 132.275 105.525) (end 133 106.25) (width 0.2) (layer "B.Cu") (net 15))
 (segment (start 132.01 106.75) (end 132.5 106.75) (width 0.2) (layer "B.Cu") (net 15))
 (segment (start 132.5 106.75) (end 133 106.25) (width 0.2) (layer "B.Cu") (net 15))
 (segment (start 138.17 113.5) (end 123 113.5) (width 0.6) (layer "F.Cu") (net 9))
 (segment (start 139.278679 111.75) (end 139.92 111.75) (width 0.2) (layer "F.Cu") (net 9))
 (segment (start 134 106.471321) (end 139.278679 111.75) (width 0.2) (layer "F.Cu") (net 9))
 (segment (start 123 113.5) (end 105.95 96.45) (width 0.6) (layer "F.Cu") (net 9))
 (segment (start 139.92 111.75) (end 138.17 113.5) (width 0.6) (layer "F.Cu") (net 9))
 (segment (start 134 104.5) (end 134 106.471321) (width 0.2) (layer "F.Cu") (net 9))
 (via (at 134 104.5) (size 0.6) (drill 0.3) (layers "F.Cu" "B.Cu") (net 9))
 (segment (start 132.275 103.95) (end 133.45 103.95) (width 0.2) (layer "B.Cu") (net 9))
 (segment (start 133.45 103.95) (end 134 104.5) (width 0.2) (layer "B.Cu") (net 9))
 (segment (start 128.25 111.75) (end 132.3 111.75) (width 0.2) (layer "F.Cu") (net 13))
 (segment (start 121 104.5) (end 128.25 111.75) (width 0.2) (layer "F.Cu") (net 13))
 (via (at 121 104.5) (size 0.6) (drill 0.3) (layers "F.Cu" "B.Cu") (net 13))
 (segment (start 122.25 103.99) (end 121.51 103.99) (width 0.2) (layer "B.Cu") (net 13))
 (segment (start 123.8625 104) (end 122.26 104) (width 0.2) (layer "B.Cu") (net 13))
 (segment (start 121.51 103.99) (end 121 104.5) (width 0.2) (layer "B.Cu") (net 13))
 (segment (start 122.26 104) (end 122.25 103.99) (width 0.2) (layer "B.Cu") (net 13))
 (segment (start 125 102.25) (end 113.25 90.5) (width 0.2) (layer "B.Cu") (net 17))
 (segment (start 125.475001 104.95) (end 125 104.474999) (width 0.2) (layer "B.Cu") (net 17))
 (segment (start 125 104.474999) (end 125 102.25) (width 0.2) (layer "B.Cu") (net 17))
 (segment (start 113.25 90.5) (end 109.75 90.5) (width 0.2) (layer "B.Cu") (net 17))
 (segment (start 126.1375 104.95) (end 125.475001 104.95) (width 0.2) (layer "B.Cu") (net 17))
 (segment (start 123.8625 103.05) (end 119.31 103.05) (width 0.2) (layer "B.Cu") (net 18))
 (segment (start 119.31 103.05) (end 109.76 93.5) (width 0.2) (layer "B.Cu") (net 18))
 (segment (start 142.1 109.25) (end 143.5 107.85) (width 0.2) (layer "B.Cu") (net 5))
 (segment (start 130 106.698924) (end 132.551076 109.25) (width 0.2) (layer "B.Cu") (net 5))
 (segment (start 132.551076 109.25) (end 142.1 109.25) (width 0.2) (layer "B.Cu") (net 5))
 (segment (start 130 104.9) (end 130 106.698924) (width 0.2) (layer "B.Cu") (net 5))
 (segment (start 130 103) (end 114.5 87.5) (width 0.2) (layer "B.Cu") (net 19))
 (segment (start 114.5 87.5) (end 109.75 87.5) (width 0.2) (layer "B.Cu") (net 19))
 (segment (start 108.73 87.5) (end 106 87.5) (width 0.2) (layer "B.Cu") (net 12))
 (segment (start 106 87.5) (end 105.95 87.45) (width 0.2) (layer "B.Cu") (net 12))
 (segment (start 106 90.5) (end 105.95 90.45) (width 0.2) (layer "B.Cu") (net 11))
 (segment (start 108.73 90.5) (end 106 90.5) (width 0.2) (layer "B.Cu") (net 11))
 (segment (start 106 93.5) (end 105.95 93.45) (width 0.2) (layer "B.Cu") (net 10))
 (segment (start 108.74 93.5) (end 106 93.5) (width 0.2) (layer "B.Cu") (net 10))
 (segment (start 151.5 107.85) (end 151.5 110.63) (width 0.2) (layer "B.Cu") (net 1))
 (segment (start 151.5 110.63) (end 152.62 111.75) (width 0.2) (layer "B.Cu") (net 1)))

